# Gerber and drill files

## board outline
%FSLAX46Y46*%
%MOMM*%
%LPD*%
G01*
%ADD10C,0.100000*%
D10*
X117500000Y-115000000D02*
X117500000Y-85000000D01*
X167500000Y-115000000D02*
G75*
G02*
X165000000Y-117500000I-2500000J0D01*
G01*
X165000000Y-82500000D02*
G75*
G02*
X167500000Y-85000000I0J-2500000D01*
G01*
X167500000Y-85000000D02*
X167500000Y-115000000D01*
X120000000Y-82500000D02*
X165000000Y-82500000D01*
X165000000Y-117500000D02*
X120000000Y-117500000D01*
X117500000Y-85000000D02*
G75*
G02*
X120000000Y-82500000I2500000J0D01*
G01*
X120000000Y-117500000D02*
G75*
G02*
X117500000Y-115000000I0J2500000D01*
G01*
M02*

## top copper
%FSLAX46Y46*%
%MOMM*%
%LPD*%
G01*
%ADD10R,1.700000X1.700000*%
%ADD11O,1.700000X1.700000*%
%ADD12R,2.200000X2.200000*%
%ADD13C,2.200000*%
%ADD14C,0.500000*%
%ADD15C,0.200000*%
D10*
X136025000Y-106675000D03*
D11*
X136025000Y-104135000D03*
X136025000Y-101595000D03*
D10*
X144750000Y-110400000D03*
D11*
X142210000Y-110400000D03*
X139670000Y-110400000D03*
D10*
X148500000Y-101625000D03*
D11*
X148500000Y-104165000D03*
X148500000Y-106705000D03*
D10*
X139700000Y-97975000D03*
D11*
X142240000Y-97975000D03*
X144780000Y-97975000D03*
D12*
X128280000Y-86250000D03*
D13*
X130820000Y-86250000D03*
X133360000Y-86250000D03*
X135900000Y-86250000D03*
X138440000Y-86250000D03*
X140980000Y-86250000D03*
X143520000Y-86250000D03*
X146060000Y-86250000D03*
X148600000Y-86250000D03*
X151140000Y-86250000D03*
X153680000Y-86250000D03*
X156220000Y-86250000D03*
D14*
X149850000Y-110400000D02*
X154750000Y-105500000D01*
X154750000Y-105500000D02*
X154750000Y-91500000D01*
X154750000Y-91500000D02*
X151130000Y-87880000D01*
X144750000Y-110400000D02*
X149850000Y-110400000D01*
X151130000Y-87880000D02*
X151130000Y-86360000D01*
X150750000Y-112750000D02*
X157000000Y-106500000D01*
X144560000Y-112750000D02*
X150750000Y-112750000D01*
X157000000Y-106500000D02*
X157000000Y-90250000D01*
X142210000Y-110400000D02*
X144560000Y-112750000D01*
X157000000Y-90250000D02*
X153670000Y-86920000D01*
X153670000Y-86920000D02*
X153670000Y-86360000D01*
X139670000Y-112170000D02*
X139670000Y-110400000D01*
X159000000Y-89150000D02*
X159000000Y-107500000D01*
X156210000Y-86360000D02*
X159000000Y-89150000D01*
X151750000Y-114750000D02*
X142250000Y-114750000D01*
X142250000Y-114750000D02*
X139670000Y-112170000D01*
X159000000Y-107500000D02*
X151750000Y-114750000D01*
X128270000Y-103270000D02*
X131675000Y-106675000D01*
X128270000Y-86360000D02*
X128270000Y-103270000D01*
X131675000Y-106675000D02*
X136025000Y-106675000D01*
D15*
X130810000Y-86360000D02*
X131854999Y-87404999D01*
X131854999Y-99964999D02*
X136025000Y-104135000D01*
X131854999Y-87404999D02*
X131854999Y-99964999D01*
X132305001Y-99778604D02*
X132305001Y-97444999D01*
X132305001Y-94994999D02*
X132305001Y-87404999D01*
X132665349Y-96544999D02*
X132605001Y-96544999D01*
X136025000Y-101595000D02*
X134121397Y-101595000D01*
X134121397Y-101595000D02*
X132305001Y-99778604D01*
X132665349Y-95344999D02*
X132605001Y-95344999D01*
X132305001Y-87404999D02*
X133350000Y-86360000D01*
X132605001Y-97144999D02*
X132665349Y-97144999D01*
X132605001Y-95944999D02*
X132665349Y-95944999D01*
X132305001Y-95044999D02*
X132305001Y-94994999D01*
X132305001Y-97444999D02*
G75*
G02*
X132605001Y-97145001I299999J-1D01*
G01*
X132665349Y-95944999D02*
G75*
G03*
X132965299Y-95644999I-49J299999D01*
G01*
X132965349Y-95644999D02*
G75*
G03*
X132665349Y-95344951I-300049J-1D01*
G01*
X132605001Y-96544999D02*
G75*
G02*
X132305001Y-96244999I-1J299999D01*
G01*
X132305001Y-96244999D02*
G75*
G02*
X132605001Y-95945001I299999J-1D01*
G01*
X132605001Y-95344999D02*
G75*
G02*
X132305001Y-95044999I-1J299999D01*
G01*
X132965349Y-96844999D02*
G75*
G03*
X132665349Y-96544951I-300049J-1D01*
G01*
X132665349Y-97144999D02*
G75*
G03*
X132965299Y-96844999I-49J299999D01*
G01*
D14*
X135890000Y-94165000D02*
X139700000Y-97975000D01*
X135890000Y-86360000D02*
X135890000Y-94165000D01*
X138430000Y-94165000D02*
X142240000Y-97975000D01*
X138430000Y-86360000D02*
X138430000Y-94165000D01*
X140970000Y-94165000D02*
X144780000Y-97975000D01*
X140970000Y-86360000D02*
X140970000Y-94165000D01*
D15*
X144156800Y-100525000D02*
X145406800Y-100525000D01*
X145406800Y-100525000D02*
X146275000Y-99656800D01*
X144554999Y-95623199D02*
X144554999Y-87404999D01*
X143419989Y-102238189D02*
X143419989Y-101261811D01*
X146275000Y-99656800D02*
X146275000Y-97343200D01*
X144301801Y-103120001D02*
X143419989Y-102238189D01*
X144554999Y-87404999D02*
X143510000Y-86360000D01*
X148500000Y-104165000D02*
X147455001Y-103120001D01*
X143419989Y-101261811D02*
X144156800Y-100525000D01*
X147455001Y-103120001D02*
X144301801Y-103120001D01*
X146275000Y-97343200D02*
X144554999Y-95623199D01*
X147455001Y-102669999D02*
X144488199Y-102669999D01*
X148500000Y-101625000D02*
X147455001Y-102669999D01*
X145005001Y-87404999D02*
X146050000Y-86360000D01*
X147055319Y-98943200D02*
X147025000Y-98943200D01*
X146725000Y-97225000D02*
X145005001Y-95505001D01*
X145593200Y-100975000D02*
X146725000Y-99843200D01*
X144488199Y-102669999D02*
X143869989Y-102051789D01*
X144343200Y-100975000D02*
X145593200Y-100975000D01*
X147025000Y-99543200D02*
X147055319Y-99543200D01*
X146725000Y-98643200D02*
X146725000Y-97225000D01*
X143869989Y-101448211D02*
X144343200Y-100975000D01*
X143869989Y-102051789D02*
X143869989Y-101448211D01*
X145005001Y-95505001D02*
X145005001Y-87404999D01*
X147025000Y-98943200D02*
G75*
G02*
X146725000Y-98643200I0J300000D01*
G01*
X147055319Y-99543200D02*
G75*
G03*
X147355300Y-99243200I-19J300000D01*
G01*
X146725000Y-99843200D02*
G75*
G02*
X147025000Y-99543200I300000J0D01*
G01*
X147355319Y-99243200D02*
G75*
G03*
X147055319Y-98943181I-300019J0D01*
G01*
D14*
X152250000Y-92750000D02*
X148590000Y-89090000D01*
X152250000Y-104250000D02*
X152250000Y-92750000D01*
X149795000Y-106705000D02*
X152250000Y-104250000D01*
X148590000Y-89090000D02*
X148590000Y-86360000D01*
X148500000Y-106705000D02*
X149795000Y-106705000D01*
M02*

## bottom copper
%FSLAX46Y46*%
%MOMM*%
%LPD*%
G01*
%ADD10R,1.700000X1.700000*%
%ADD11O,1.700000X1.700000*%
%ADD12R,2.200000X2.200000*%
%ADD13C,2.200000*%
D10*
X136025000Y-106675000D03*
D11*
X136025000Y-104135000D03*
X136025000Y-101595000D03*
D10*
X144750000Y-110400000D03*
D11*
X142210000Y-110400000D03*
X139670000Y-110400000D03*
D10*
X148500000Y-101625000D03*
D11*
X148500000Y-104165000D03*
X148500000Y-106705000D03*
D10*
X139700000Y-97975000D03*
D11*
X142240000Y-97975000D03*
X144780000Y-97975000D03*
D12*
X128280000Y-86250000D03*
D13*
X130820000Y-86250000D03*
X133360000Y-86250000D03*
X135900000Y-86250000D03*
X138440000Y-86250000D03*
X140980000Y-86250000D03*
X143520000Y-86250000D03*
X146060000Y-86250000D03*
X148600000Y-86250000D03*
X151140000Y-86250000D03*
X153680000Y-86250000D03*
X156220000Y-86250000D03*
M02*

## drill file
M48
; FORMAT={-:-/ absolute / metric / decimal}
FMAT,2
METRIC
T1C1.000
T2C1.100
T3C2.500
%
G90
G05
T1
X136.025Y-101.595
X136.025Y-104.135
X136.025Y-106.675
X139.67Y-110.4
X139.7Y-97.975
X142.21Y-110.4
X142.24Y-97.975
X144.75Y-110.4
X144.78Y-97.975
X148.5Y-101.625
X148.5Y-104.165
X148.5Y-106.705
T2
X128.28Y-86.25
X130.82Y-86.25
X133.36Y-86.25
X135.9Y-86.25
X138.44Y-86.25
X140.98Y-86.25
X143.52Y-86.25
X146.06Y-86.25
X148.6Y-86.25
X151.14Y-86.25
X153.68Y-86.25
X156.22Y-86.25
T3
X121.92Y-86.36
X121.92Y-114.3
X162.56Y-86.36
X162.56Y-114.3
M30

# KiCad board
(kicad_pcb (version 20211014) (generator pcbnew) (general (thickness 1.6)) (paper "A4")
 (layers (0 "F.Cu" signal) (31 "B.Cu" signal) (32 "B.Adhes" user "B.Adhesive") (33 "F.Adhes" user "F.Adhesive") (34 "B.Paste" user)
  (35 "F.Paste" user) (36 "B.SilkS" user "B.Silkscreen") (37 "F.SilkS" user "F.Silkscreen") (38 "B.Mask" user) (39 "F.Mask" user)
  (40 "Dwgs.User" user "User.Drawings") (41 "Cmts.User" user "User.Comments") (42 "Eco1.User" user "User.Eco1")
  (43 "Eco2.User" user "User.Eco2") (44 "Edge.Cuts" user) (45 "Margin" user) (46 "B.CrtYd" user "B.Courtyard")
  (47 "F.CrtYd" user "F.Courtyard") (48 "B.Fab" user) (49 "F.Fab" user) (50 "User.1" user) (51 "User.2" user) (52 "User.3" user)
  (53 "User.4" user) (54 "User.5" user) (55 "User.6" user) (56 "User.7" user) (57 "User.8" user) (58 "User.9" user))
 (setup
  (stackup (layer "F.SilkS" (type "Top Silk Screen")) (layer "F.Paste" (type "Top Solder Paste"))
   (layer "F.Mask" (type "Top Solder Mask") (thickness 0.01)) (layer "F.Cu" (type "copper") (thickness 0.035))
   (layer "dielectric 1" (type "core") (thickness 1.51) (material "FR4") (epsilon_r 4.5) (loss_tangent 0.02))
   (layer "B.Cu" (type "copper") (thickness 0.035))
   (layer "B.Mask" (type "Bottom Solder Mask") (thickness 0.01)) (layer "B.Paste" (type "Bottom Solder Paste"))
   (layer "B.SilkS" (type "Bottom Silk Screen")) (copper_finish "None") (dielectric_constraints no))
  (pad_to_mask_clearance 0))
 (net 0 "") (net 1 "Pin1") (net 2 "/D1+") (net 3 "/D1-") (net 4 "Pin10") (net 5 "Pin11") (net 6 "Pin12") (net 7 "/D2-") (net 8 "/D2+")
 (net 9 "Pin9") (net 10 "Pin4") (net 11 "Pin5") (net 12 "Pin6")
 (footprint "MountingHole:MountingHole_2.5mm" (layer "F.Cu") (at 162.56 114.3)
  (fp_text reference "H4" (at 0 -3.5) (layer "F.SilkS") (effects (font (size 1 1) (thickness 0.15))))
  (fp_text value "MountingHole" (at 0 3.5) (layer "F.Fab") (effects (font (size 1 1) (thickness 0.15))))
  (pad "" np_thru_hole circle (at 0 0) (size 2.5 2.5) (drill 2.5) (layers *.Cu *.Mask)))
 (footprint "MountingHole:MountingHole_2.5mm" (layer "F.Cu") (at 162.56 86.36)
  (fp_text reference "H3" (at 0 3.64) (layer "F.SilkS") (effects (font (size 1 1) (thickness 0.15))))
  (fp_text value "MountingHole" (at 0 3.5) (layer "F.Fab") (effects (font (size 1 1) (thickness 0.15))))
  (pad "" np_thru_hole circle (at 0 0) (size 2.5 2.5) (drill 2.5) (layers *.Cu *.Mask)))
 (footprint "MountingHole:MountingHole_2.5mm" (layer "F.Cu") (at 121.92 114.3)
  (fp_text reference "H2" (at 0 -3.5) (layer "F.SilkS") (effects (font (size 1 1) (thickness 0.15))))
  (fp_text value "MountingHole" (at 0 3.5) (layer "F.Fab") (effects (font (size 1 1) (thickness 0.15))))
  (pad "" np_thru_hole circle (at 0 0) (size 2.5 2.5) (drill 2.5) (layers *.Cu *.Mask)))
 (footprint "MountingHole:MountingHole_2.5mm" (layer "F.Cu") (at 121.92 86.36)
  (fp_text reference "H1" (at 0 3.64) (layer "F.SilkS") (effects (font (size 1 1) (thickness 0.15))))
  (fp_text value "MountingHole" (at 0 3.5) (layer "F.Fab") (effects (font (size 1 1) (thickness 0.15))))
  (pad "" np_thru_hole circle (at 0 0) (size 2.5 2.5) (drill 2.5) (layers *.Cu *.Mask)))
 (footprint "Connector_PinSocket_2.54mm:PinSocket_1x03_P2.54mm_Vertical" (layer "F.Cu") (at 136.025 106.675 180)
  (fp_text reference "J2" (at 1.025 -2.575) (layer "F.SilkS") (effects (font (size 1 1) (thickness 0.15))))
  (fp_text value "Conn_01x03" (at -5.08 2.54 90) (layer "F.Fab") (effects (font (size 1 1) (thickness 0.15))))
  (pad "1" thru_hole rect (at 0 0 180) (size 1.7 1.7) (drill 1) (layers *.Cu *.Mask) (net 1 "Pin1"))
  (pad "2" thru_hole oval (at 0 2.54 180) (size 1.7 1.7) (drill 1) (layers *.Cu *.Mask) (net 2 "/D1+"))
  (pad "3" thru_hole oval (at 0 5.08 180) (size 1.7 1.7) (drill 1) (layers *.Cu *.Mask) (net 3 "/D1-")))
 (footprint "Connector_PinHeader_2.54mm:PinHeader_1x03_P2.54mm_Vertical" (layer "F.Cu") (at 144.75 110.4 -90)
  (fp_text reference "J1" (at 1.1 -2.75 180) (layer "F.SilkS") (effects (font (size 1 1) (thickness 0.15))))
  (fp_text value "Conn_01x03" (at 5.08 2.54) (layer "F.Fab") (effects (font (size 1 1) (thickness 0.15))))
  (pad "1" thru_hole rect (at 0 0 270) (size 1.7 1.7) (drill 1) (layers *.Cu *.Mask) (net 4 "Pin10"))
  (pad "2" thru_hole oval (at 0 2.54 270) (size 1.7 1.7) (drill 1) (layers *.Cu *.Mask) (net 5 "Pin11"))
  (pad "3" thru_hole oval (at 0 5.08 270) (size 1.7 1.7) (drill 1) (layers *.Cu *.Mask) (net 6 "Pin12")))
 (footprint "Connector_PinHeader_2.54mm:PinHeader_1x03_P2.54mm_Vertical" (layer "F.Cu") (at 148.5 101.625)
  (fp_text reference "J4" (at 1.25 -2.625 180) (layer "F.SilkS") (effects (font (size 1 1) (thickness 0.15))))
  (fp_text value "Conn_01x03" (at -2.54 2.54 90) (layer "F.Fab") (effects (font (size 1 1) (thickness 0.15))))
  (pad "1" thru_hole rect (at 0 0) (size 1.7 1.7) (drill 1) (layers *.Cu *.Mask) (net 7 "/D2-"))
  (pad "2" thru_hole oval (at 0 2.54) (size 1.7 1.7) (drill 1) (layers *.Cu *.Mask) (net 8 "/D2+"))
  (pad "3" thru_hole oval (at 0 5.08) (size 1.7 1.7) (drill 1) (layers *.Cu *.Mask) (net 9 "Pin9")))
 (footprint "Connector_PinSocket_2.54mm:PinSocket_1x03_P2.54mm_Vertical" (layer "F.Cu") (at 139.7 97.975 90)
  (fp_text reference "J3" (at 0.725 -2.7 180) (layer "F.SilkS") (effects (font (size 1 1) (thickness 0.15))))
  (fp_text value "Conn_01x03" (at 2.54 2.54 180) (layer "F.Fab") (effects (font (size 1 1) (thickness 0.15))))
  (pad "1" thru_hole rect (at 0 0 90) (size 1.7 1.7) (drill 1) (layers *.Cu *.Mask) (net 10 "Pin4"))
  (pad "2" thru_hole oval (at 0 2.54 90) (size 1.7 1.7) (drill 1) (layers *.Cu *.Mask) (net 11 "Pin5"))
  (pad "3" thru_hole oval (at 0 5.08 90) (size 1.7 1.7) (drill 1) (layers *.Cu *.Mask) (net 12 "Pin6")))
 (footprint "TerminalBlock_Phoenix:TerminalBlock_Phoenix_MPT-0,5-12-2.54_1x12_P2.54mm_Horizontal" (layer "B.Cu") (at 128.28 86.25)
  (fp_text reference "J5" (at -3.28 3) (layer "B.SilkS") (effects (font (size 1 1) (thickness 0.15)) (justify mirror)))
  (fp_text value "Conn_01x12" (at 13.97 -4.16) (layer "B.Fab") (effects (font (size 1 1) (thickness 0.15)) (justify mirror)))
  (pad "1" thru_hole rect (at 0 0) (size 2.2 2.2) (drill 1.1) (layers *.Cu *.Mask) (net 1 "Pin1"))
  (pad "2" thru_hole circle (at 2.54 0) (size 2.2 2.2) (drill 1.1) (layers *.Cu *.Mask) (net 2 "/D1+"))
  (pad "3" thru_hole circle (at 5.08 0) (size 2.2 2.2) (drill 1.1) (layers *.Cu *.Mask) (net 3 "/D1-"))
  (pad "4" thru_hole circle (at 7.62 0) (size 2.2 2.2) (drill 1.1) (layers *.Cu *.Mask) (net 10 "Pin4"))
  (pad "5" thru_hole circle (at 10.16 0) (size 2.2 2.2) (drill 1.1) (layers *.Cu *.Mask) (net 11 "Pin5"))
  (pad "6" thru_hole circle (at 12.7 0) (size 2.2 2.2) (drill 1.1) (layers *.Cu *.Mask) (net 12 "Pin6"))
  (pad "7" thru_hole circle (at 15.24 0) (size 2.2 2.2) (drill 1.1) (layers *.Cu *.Mask) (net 8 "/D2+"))
  (pad "8" thru_hole circle (at 17.78 0) (size 2.2 2.2) (drill 1.1) (layers *.Cu *.Mask) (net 7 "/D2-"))
  (pad "9" thru_hole circle (at 20.32 0) (size 2.2 2.2) (drill 1.1) (layers *.Cu *.Mask) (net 9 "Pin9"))
  (pad "10" thru_hole circle (at 22.86 0) (size 2.2 2.2) (drill 1.1) (layers *.Cu *.Mask) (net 4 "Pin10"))
  (pad "11" thru_hole circle (at 25.4 0) (size 2.2 2.2) (drill 1.1) (layers *.Cu *.Mask) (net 5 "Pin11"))
  (pad "12" thru_hole circle (at 27.94 0) (size 2.2 2.2) (drill 1.1) (layers *.Cu *.Mask) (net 6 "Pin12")))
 (gr_line (start 117.5 115) (end 117.5 85) (layer "Edge.Cuts") (width 0.1))
 (gr_arc (start 167.5 115) (mid 166.767767 116.767767) (end 165 117.5) (layer "Edge.Cuts") (width 0.1))
 (gr_arc (start 165 82.5) (mid 166.767767 83.232233) (end 167.5 85) (layer "Edge.Cuts") (width 0.1))
 (gr_line (start 167.5 85) (end 167.5 115) (layer "Edge.Cuts") (width 0.1))
 (gr_line (start 120 82.5) (end 165 82.5) (layer "Edge.Cuts") (width 0.1))
 (gr_line (start 165 117.5) (end 120 117.5) (layer "Edge.Cuts") (width 0.1))
 (gr_arc (start 117.5 85) (mid 118.232233 83.232233) (end 120 82.5) (layer "Edge.Cuts") (width 0.1))
 (gr_arc (start 120 117.5) (mid 118.232233 116.767767) (end 117.5 115) (layer "Edge.Cuts") (width 0.1))
 (segment (start 149.85 110.4) (end 154.75 105.5) (width 0.5) (layer "F.Cu") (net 4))
 (segment (start 154.75 105.5) (end 154.75 91.5) (width 0.5) (layer "F.Cu") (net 4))
 (segment (start 154.75 91.5) (end 151.13 87.88) (width 0.5) (layer "F.Cu") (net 4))
 (segment (start 144.75 110.4) (end 149.85 110.4) (width 0.5) (layer "F.Cu") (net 4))
 (segment (start 151.13 87.88) (end 151.13 86.36) (width 0.5) (layer "F.Cu") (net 4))
 (segment (start 150.75 112.75) (end 157 106.5) (width 0.5) (layer "F.Cu") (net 5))
 (segment (start 144.56 112.75) (end 150.75 112.75) (width 0.5) (layer "F.Cu") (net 5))
 (segment (start 157 106.5) (end 157 90.25) (width 0.5) (layer "F.Cu") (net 5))
 (segment (start 142.21 110.4) (end 144.56 112.75) (width 0.5) (layer "F.Cu") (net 5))
 (segment (start 157 90.25) (end 153.67 86.92) (width 0.5) (layer "F.Cu") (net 5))
 (segment (start 153.67 86.92) (end 153.67 86.36) (width 0.5) (layer "F.Cu") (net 5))
 (segment (start 139.67 112.17) (end 139.67 110.4) (width 0.5) (layer "F.Cu") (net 6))
 (segment (start 159 89.15) (end 159 107.5) (width 0.5) (layer "F.Cu") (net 6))
 (segment (start 156.21 86.36) (end 159 89.15) (width 0.5) (layer "F.Cu") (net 6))
 (segment (start 151.75 114.75) (end 142.25 114.75) (width 0.5) (layer "F.Cu") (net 6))
 (segment (start 142.25 114.75) (end 139.67 112.17) (width 0.5) (layer "F.Cu") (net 6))
 (segment (start 159 107.5) (end 151.75 114.75) (width 0.5) (layer "F.Cu") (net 6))
 (segment (start 128.27 103.27) (end 131.675 106.675) (width 0.5) (layer "F.Cu") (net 1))
 (segment (start 128.27 86.36) (end 128.27 103.27) (width 0.5) (layer "F.Cu") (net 1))
 (segment (start 131.675 106.675) (end 136.025 106.675) (width 0.5) (layer "F.Cu") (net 1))
 (segment (start 130.81 86.36) (end 131.854999 87.404999) (width 0.2) (layer "F.Cu") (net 2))
 (segment (start 131.854999 99.964999) (end 136.025 104.135) (width 0.2) (layer "F.Cu") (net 2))
 (segment (start 131.854999 87.404999) (end 131.854999 99.964999) (width 0.2) (layer "F.Cu") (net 2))
 (segment (start 132.305001 99.778604) (end 132.305001 97.444999) (width 0.2) (layer "F.Cu") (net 3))
 (segment (start 132.305001 94.994999) (end 132.305001 87.404999) (width 0.2) (layer "F.Cu") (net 3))
 (segment (start 132.665349 96.544999) (end 132.605001 96.544999) (width 0.2) (layer "F.Cu") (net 3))
 (segment (start 136.025 101.595) (end 134.121397 101.595) (width 0.2) (layer "F.Cu") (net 3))
 (segment (start 134.121397 101.595) (end 132.305001 99.778604) (width 0.2) (layer "F.Cu") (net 3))
 (segment (start 132.665349 95.344999) (end 132.605001 95.344999) (width 0.2) (layer "F.Cu") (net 3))
 (segment (start 132.305001 87.404999) (end 133.35 86.36) (width 0.2) (layer "F.Cu") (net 3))
 (segment (start 132.605001 97.144999) (end 132.665349 97.144999) (width 0.2) (layer "F.Cu") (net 3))
 (segment (start 132.605001 95.944999) (end 132.665349 95.944999) (width 0.2) (layer "F.Cu") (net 3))
 (segment (start 132.305001 95.044999) (end 132.305001 94.994999) (width 0.2) (layer "F.Cu") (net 3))
 (arc (start 132.305001 97.444999) (mid 132.392869 97.232867) (end 132.605001 97.144999) (width 0.2) (layer "F.Cu") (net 3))
 (arc (start 132.665349 95.944999) (mid 132.877481 95.857131) (end 132.965349 95.644999) (width 0.2) (layer "F.Cu") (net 3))
 (arc (start 132.965349 95.644999) (mid 132.877481 95.432867) (end 132.665349 95.344999) (width 0.2) (layer "F.Cu") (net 3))
 (arc (start 132.605001 96.544999) (mid 132.392869 96.457131) (end 132.305001 96.244999) (width 0.2) (layer "F.Cu") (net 3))
 (arc (start 132.305001 96.244999) (mid 132.392869 96.032867) (end 132.605001 95.944999) (width 0.2) (layer "F.Cu") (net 3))
 (arc (start 132.605001 95.344999) (mid 132.392869 95.257131) (end 132.305001 95.044999) (width 0.2) (layer "F.Cu") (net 3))
 (arc (start 132.965349 96.844999) (mid 132.877481 96.632867) (end 132.665349 96.544999) (width 0.2) (layer "F.Cu") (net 3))
 (arc (start 132.665349 97.144999) (mid 132.877481 97.057131) (end 132.965349 96.844999) (width 0.2) (layer "F.Cu") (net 3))
 (segment (start 135.89 94.165) (end 139.7 97.975) (width 0.5) (layer "F.Cu") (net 10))
 (segment (start 135.89 86.36) (end 135.89 94.165) (width 0.5) (layer "F.Cu") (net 10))
 (segment (start 138.43 94.165) (end 142.24 97.975) (width 0.5) (layer "F.Cu") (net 11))
 (segment (start 138.43 86.36) (end 138.43 94.165) (width 0.5) (layer "F.Cu") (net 11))
 (segment (start 140.97 94.165) (end 144.78 97.975) (width 0.5) (layer "F.Cu") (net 12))
 (segment (start 140.97 86.36) (end 140.97 94.165) (width 0.5) (layer "F.Cu") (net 12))
 (segment (start 144.1568 100.525) (end 145.4068 100.525) (width 0.2) (layer "F.Cu") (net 8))
 (segment (start 145.4068 100.525) (end 146.275 99.6568) (width 0.2) (layer "F.Cu") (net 8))
 (segment (start 144.554999 95.623199) (end 144.554999 87.404999) (width 0.2) (layer "F.Cu") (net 8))
 (segment (start 143.419989 102.238189) (end 143.419989 101.261811) (width 0.2) (layer "F.Cu") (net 8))
 (segment (start 146.275 99.6568) (end 146.275 97.3432) (width 0.2) (layer "F.Cu") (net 8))
 (segment (start 144.301801 103.120001) (end 143.419989 102.238189) (width 0.2) (layer "F.Cu") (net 8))
 (segment (start 144.554999 87.404999) (end 143.51 86.36) (width 0.2) (layer "F.Cu") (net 8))
 (segment (start 148.5 104.165) (end 147.455001 103.120001) (width 0.2) (layer "F.Cu") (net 8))
 (segment (start 143.419989 101.261811) (end 144.1568 100.525) (width 0.2) (layer "F.Cu") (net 8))
 (segment (start 147.455001 103.120001) (end 144.301801 103.120001) (width 0.2) (layer "F.Cu") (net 8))
 (segment (start 146.275 97.3432) (end 144.554999 95.623199) (width 0.2) (layer "F.Cu") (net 8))
 (segment (start 147.455001 102.669999) (end 144.488199 102.669999) (width 0.2) (layer "F.Cu") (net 7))
 (segment (start 148.5 101.625) (end 147.455001 102.669999) (width 0.2) (layer "F.Cu") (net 7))
 (segment (start 145.005001 87.404999) (end 146.05 86.36) (width 0.2) (layer "F.Cu") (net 7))
 (segment (start 147.055319 98.9432) (end 147.025 98.9432) (width 0.2) (layer "F.Cu") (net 7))
 (segment (start 146.725 97.225) (end 145.005001 95.505001) (width 0.2) (layer "F.Cu") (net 7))
 (segment (start 145.5932 100.975) (end 146.725 99.8432) (width 0.2) (layer "F.Cu") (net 7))
 (segment (start 144.488199 102.669999) (end 143.869989 102.051789) (width 0.2) (layer "F.Cu") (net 7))
 (segment (start 144.3432 100.975) (end 145.5932 100.975) (width 0.2) (layer "F.Cu") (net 7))
 (segment (start 147.025 99.5432) (end 147.055319 99.5432) (width 0.2) (layer "F.Cu") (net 7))
 (segment (start 146.725 98.6432) (end 146.725 97.225) (width 0.2) (layer "F.Cu") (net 7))
 (segment (start 143.869989 101.448211) (end 144.3432 100.975) (width 0.2) (layer "F.Cu") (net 7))
 (segment (start 143.869989 102.051789) (end 143.869989 101.448211) (width 0.2) (layer "F.Cu") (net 7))
 (segment (start 145.005001 95.505001) (end 145.005001 87.404999) (width 0.2) (layer "F.Cu") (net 7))
 (arc (start 147.025 98.9432) (mid 146.812868 98.855332) (end 146.725 98.6432) (width 0.2) (layer "F.Cu") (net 7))
 (arc (start 147.055319 99.5432) (mid 147.267451 99.455332) (end 147.355319 99.2432) (width 0.2) (layer "F.Cu") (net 7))
 (arc (start 146.725 99.8432) (mid 146.812868 99.631068) (end 147.025 99.5432) (width 0.2) (layer "F.Cu") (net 7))
 (arc (start 147.355319 99.2432) (mid 147.267451 99.031068) (end 147.055319 98.9432) (width 0.2) (layer "F.Cu") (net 7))
 (segment (start 152.25 92.75) (end 148.59 89.09) (width 0.5) (layer "F.Cu") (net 9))
 (segment (start 152.25 104.25) (end 152.25 92.75) (width 0.5) (layer "F.Cu") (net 9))
 (segment (start 149.795 106.705) (end 152.25 104.25) (width 0.5) (layer "F.Cu") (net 9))
 (segment (start 148.59 89.09) (end 148.59 86.36) (width 0.5) (layer "F.Cu") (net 9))
 (segment (start 148.5 106.705) (end 149.795 106.705) (width 0.5) (layer "F.Cu") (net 9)))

